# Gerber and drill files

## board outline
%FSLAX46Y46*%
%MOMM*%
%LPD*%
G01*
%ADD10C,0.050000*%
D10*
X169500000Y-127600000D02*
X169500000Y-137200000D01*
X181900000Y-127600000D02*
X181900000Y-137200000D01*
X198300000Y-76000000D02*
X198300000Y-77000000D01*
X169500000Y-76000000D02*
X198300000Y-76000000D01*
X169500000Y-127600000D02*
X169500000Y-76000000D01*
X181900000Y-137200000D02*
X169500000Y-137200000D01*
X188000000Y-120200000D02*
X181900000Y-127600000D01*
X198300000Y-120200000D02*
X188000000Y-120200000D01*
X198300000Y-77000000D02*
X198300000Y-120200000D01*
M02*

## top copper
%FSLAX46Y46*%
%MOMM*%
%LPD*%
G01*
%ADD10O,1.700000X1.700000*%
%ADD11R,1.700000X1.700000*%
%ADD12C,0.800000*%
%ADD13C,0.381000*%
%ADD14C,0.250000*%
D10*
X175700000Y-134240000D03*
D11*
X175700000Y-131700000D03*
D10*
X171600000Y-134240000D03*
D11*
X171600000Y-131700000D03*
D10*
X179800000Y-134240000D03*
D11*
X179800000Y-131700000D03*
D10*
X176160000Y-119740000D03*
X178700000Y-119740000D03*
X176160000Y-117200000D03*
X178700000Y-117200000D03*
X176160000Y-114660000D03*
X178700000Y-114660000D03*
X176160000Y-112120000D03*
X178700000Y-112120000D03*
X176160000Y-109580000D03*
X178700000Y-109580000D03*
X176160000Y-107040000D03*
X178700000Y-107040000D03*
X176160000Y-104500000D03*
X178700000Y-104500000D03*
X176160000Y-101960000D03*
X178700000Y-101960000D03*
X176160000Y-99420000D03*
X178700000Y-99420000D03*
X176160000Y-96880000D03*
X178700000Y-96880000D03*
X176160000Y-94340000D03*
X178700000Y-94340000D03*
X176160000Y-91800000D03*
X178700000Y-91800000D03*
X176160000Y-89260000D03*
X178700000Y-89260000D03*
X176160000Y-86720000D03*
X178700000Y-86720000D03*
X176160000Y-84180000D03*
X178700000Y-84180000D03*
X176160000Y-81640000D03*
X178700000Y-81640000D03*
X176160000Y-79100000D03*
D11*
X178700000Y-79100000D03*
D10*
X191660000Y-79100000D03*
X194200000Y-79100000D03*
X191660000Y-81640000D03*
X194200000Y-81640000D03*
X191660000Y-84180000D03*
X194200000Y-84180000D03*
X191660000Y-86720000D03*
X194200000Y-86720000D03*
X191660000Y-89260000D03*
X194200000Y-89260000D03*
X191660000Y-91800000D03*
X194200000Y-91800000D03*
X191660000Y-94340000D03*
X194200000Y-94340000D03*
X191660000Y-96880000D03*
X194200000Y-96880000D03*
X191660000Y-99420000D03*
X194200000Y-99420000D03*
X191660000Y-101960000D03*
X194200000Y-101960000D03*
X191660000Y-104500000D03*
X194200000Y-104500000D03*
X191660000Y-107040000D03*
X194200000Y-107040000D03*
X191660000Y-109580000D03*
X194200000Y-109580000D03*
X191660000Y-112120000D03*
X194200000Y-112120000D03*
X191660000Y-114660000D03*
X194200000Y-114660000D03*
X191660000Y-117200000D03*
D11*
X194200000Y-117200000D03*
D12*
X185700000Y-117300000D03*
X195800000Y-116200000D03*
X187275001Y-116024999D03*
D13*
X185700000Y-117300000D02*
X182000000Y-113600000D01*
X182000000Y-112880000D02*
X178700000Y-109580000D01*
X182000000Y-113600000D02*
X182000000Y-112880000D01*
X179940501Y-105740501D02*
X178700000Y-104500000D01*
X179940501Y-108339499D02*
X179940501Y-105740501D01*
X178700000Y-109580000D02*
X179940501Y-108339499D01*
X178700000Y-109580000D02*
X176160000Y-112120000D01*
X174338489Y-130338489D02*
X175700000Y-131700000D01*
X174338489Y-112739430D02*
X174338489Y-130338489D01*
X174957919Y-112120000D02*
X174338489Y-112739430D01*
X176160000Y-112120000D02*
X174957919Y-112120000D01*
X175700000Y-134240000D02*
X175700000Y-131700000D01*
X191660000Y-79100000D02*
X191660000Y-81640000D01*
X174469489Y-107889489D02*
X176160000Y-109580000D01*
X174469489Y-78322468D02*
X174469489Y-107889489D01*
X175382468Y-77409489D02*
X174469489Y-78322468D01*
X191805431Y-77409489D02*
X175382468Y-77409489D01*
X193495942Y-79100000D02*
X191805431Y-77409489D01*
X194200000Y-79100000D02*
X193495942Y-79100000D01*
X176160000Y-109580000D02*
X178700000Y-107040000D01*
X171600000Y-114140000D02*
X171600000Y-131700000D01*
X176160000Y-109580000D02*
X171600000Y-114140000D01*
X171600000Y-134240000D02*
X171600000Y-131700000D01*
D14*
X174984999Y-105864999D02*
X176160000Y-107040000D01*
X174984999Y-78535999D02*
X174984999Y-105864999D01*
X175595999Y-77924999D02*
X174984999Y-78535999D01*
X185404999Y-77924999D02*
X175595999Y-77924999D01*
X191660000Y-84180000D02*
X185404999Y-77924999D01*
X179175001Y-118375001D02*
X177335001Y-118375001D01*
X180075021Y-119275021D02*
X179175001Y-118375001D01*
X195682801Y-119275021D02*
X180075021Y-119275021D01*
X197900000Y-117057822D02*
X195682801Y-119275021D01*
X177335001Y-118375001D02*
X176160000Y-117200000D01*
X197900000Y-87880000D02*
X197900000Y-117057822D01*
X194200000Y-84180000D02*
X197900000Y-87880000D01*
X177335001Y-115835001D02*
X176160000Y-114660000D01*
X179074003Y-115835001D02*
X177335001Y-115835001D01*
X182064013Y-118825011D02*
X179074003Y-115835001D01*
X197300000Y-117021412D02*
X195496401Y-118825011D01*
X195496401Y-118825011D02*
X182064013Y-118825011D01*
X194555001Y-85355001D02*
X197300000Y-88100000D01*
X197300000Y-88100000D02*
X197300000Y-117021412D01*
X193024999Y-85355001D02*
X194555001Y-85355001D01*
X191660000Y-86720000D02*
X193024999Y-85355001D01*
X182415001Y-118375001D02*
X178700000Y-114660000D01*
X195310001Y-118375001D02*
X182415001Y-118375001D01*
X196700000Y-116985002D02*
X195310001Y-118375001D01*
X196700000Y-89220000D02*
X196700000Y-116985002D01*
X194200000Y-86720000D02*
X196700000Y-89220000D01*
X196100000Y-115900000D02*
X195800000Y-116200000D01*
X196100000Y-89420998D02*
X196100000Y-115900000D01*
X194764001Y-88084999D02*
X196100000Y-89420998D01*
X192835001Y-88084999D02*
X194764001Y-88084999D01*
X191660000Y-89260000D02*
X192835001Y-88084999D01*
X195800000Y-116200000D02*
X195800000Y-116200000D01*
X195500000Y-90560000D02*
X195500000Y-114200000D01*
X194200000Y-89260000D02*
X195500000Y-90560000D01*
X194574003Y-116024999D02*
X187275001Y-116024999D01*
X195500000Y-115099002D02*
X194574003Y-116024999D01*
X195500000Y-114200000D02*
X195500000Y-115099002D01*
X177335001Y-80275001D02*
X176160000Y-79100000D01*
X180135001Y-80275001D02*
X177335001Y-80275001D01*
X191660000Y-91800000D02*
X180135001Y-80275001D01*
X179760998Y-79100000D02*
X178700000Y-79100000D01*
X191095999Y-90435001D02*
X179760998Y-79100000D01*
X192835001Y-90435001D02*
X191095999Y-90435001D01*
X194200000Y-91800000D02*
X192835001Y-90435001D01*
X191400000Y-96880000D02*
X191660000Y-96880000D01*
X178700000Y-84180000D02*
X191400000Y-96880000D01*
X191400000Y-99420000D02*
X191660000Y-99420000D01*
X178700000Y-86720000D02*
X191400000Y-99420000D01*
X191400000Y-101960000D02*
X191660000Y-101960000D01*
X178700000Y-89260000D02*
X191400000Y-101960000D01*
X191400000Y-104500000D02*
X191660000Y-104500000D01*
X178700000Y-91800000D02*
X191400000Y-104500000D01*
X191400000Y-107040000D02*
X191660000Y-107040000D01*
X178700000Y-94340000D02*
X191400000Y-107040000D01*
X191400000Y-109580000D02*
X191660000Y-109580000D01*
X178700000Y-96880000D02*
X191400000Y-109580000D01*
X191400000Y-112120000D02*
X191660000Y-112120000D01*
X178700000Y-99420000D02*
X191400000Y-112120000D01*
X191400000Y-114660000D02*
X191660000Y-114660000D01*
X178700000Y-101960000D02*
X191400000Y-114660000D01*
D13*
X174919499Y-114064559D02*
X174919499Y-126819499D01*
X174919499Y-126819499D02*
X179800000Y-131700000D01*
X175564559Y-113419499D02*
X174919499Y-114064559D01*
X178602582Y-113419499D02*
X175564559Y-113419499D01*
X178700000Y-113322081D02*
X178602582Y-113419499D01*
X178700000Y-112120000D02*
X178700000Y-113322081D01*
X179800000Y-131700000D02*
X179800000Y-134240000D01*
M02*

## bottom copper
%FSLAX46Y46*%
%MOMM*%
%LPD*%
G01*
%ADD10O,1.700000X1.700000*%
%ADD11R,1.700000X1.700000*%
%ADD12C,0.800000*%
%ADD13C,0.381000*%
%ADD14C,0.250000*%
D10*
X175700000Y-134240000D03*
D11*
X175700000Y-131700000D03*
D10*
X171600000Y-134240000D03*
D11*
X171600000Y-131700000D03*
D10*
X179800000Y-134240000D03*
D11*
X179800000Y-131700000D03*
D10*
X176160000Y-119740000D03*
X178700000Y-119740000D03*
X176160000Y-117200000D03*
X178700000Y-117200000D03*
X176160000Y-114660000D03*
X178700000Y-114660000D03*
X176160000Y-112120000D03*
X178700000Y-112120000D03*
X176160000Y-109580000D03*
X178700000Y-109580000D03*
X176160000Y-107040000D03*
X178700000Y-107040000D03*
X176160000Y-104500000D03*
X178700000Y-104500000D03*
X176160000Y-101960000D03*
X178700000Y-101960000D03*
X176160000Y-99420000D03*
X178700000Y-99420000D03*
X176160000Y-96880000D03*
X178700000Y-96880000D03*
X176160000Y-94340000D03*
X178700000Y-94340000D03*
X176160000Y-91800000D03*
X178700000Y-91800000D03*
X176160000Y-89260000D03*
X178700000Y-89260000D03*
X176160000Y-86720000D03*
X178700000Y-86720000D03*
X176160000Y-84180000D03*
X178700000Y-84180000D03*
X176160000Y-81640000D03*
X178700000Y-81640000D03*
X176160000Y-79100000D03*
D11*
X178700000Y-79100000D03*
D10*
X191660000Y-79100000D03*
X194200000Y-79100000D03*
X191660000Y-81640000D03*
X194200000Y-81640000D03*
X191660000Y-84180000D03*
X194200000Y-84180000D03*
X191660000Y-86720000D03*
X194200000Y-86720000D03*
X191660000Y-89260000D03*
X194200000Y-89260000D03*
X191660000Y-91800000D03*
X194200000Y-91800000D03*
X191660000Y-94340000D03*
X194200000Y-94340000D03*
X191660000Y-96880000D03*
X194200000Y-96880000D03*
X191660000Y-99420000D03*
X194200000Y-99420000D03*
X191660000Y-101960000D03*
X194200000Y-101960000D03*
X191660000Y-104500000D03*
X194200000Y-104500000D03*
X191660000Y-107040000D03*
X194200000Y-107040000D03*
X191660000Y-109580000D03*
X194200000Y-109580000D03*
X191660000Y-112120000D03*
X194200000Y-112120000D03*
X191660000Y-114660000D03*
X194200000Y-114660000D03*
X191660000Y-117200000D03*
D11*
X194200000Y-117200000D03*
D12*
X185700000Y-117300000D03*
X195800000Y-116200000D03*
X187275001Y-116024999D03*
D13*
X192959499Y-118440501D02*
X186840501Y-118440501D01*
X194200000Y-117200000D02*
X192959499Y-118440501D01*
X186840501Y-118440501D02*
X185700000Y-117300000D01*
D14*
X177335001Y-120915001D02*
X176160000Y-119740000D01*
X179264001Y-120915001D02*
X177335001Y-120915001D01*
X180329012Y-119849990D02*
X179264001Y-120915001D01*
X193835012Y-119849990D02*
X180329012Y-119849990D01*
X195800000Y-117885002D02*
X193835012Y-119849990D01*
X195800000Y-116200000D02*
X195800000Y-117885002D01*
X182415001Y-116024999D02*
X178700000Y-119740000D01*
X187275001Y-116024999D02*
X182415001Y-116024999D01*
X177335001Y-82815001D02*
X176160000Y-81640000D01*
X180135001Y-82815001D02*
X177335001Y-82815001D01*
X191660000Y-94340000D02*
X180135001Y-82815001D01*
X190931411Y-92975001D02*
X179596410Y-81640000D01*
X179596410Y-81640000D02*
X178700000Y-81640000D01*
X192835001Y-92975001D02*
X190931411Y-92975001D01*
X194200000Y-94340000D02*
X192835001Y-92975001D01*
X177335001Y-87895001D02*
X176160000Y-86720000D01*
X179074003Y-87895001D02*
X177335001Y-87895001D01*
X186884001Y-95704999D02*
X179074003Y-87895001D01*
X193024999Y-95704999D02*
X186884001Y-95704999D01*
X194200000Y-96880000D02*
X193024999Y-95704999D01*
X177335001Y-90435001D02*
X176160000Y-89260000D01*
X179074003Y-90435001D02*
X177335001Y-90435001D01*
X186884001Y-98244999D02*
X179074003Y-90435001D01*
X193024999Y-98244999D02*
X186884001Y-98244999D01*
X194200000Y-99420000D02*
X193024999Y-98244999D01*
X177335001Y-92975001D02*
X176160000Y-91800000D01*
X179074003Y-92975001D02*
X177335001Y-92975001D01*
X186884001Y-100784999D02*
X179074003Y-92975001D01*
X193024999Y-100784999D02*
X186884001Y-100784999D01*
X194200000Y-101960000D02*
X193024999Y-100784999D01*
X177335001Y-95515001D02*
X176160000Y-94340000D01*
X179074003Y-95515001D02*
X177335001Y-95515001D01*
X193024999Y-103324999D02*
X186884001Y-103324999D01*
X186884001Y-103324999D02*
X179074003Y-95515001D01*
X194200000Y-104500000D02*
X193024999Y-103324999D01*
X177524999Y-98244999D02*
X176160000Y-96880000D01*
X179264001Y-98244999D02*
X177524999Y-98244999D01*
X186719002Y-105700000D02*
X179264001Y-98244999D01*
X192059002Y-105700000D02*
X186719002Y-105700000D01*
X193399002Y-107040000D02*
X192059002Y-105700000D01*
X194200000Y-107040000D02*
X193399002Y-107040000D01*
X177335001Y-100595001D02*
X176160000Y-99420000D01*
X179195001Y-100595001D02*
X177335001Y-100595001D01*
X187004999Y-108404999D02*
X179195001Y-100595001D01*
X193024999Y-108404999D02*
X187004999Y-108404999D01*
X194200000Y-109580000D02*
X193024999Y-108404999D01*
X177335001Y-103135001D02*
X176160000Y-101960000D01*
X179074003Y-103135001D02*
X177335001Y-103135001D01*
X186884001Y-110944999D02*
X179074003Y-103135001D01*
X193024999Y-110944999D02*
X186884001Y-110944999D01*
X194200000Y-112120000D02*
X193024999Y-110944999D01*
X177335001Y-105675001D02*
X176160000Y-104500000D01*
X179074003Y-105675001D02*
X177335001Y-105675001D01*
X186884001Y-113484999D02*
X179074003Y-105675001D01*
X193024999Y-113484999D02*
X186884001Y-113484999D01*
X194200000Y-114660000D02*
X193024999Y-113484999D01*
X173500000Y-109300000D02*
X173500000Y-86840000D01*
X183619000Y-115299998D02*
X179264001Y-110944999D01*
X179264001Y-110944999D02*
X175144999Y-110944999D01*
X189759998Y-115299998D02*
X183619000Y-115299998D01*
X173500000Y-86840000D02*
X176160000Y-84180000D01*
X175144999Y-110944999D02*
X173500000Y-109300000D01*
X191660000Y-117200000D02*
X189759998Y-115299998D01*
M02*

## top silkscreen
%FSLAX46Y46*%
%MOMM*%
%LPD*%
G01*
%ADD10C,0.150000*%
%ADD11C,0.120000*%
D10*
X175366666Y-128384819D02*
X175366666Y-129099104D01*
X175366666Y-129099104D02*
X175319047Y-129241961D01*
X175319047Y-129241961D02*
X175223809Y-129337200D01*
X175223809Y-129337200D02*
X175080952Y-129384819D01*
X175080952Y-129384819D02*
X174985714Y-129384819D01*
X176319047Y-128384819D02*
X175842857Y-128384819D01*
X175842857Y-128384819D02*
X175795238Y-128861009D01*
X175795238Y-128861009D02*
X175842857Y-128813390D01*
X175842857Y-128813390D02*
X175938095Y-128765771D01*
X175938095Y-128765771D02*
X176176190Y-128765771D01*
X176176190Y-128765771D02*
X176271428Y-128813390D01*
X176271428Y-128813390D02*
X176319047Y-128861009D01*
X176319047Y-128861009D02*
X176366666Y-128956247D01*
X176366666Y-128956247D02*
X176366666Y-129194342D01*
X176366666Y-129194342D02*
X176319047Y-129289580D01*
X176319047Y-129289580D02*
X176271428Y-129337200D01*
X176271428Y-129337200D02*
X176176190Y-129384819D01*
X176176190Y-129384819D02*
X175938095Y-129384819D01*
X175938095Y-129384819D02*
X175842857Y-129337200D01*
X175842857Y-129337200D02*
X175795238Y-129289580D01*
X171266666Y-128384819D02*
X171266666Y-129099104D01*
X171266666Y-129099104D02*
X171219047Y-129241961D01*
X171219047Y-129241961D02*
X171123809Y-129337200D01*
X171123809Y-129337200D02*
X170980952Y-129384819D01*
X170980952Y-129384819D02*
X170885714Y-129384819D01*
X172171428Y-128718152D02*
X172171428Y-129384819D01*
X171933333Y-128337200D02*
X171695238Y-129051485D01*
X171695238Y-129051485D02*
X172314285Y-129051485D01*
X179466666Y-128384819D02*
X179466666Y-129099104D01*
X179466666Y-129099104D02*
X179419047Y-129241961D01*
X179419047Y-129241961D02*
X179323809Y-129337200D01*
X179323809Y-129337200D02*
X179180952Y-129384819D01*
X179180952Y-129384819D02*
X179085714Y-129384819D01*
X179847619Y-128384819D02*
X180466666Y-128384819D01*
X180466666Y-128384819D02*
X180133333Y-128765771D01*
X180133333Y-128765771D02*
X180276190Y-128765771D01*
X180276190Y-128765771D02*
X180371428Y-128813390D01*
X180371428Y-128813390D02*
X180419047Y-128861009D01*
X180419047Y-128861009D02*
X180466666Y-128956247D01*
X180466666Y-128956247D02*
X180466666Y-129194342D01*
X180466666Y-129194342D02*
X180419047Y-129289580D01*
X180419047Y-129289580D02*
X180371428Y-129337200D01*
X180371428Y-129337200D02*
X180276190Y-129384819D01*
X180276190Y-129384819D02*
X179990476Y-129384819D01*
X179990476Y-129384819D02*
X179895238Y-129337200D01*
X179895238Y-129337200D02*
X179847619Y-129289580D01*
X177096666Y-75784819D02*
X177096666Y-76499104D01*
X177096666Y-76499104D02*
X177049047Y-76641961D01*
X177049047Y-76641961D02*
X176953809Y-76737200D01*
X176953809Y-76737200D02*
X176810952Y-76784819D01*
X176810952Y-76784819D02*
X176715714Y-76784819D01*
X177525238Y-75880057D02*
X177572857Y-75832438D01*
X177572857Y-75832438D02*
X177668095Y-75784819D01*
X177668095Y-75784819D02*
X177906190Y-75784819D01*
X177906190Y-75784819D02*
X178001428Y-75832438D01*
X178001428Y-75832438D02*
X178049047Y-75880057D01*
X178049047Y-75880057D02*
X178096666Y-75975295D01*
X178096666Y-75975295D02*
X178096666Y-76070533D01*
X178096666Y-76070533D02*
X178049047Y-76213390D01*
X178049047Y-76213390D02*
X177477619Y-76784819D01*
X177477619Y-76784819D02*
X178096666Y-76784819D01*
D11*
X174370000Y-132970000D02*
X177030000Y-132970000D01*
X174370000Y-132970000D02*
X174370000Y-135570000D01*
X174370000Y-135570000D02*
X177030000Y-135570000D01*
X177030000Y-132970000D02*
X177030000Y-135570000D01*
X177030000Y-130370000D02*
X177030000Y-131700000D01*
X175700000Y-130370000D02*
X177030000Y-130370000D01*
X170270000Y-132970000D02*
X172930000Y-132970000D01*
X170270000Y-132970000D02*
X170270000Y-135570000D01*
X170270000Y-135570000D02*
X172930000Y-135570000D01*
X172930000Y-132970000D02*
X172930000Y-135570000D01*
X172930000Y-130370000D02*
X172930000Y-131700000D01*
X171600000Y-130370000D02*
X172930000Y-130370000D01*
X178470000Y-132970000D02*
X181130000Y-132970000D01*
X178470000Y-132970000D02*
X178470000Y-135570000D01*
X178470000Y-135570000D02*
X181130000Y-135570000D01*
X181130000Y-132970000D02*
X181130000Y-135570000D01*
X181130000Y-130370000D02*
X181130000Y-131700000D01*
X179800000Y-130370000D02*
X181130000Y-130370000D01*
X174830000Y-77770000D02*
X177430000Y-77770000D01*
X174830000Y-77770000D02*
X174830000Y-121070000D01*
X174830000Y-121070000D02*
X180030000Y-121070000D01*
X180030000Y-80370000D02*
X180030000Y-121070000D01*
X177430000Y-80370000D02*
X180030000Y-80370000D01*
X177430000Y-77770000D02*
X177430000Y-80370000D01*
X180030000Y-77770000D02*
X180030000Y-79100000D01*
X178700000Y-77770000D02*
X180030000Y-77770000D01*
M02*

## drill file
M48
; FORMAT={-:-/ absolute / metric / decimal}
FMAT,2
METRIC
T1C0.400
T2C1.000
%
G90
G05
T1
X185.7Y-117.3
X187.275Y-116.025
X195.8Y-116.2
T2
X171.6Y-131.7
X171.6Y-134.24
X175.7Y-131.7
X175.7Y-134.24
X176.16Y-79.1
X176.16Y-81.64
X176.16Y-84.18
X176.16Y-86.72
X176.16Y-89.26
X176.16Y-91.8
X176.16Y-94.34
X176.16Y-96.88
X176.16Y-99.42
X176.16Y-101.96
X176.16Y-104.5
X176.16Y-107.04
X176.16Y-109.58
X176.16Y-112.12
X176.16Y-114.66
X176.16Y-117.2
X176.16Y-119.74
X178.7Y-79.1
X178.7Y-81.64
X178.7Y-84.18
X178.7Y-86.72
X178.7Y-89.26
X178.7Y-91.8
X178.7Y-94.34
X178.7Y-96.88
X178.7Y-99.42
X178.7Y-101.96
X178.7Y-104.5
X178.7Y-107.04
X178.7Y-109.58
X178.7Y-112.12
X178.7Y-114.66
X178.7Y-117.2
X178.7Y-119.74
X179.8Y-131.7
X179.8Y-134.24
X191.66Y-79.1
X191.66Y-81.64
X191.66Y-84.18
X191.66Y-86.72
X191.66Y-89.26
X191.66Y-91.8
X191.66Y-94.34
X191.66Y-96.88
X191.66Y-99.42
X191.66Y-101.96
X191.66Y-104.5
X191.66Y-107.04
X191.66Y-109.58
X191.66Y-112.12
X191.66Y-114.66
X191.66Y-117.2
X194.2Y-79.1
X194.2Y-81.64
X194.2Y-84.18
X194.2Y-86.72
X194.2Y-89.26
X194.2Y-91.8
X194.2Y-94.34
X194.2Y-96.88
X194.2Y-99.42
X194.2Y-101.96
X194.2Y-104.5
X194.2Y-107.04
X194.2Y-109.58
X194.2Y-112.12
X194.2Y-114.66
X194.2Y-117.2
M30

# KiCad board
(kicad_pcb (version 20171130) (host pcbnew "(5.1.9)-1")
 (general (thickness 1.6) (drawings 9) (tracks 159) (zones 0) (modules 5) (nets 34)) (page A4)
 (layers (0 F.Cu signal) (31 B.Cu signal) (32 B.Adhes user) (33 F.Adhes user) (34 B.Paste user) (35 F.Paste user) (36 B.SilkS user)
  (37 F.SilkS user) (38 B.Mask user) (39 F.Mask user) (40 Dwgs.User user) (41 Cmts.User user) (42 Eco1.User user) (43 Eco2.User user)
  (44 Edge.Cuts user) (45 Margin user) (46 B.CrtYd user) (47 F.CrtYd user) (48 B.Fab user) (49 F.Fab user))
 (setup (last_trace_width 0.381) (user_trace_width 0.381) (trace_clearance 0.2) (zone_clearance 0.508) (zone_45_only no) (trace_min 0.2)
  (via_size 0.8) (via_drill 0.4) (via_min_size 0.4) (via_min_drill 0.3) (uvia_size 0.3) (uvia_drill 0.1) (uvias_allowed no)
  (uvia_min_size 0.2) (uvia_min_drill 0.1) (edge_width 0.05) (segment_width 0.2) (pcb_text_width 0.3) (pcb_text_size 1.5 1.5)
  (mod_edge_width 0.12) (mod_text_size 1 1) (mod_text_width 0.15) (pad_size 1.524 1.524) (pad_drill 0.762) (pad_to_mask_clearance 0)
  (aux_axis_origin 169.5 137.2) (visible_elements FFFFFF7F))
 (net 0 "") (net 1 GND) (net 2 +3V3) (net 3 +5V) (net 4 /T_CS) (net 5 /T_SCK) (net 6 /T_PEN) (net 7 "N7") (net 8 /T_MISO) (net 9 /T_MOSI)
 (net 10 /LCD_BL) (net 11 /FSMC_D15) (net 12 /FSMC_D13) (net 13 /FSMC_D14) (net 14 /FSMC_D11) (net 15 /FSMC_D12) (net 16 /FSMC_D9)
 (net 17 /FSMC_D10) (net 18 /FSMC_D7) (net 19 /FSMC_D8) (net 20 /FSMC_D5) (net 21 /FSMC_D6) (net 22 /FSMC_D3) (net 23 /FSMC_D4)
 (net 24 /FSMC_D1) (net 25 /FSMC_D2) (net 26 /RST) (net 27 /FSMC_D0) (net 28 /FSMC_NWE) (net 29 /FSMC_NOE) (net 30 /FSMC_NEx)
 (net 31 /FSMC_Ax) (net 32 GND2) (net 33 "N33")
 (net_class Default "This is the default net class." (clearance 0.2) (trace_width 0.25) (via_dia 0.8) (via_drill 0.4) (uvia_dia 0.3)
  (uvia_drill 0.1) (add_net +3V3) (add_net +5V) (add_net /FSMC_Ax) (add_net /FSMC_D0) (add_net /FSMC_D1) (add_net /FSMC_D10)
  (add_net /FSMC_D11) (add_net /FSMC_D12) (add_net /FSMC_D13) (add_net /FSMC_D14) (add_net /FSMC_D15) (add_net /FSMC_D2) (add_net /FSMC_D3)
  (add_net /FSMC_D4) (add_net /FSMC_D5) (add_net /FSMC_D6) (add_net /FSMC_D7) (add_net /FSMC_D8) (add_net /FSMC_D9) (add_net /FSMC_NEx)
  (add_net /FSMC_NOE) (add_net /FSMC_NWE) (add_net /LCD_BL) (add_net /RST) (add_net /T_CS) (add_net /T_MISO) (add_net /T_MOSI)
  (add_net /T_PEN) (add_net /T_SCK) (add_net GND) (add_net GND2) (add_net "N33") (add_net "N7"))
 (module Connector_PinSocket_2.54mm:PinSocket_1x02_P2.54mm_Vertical (layer F.Cu) (at 175.7 131.7)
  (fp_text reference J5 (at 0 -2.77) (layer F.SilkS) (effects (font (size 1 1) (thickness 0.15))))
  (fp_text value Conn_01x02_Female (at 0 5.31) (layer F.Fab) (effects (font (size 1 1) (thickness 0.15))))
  (fp_line (start -1.33 1.27) (end 1.33 1.27) (layer F.SilkS) (width 0.12))
  (fp_line (start -1.33 1.27) (end -1.33 3.87) (layer F.SilkS) (width 0.12))
  (fp_line (start -1.33 3.87) (end 1.33 3.87) (layer F.SilkS) (width 0.12))
  (fp_line (start 1.33 1.27) (end 1.33 3.87) (layer F.SilkS) (width 0.12))
  (fp_line (start 1.33 -1.33) (end 1.33 0) (layer F.SilkS) (width 0.12))
  (fp_line (start 0 -1.33) (end 1.33 -1.33) (layer F.SilkS) (width 0.12))
  (pad 2 thru_hole oval (at 0 2.54) (size 1.7 1.7) (drill 1) (layers *.Cu *.Mask) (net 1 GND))
  (pad 1 thru_hole rect (at 0 0) (size 1.7 1.7) (drill 1) (layers *.Cu *.Mask) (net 1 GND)))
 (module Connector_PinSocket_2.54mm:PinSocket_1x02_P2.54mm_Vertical (layer F.Cu) (at 171.6 131.7)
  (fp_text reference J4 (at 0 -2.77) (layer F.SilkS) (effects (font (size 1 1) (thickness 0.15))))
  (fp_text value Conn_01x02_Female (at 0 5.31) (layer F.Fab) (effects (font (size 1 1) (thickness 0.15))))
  (fp_line (start -1.33 1.27) (end 1.33 1.27) (layer F.SilkS) (width 0.12))
  (fp_line (start -1.33 1.27) (end -1.33 3.87) (layer F.SilkS) (width 0.12))
  (fp_line (start -1.33 3.87) (end 1.33 3.87) (layer F.SilkS) (width 0.12))
  (fp_line (start 1.33 1.27) (end 1.33 3.87) (layer F.SilkS) (width 0.12))
  (fp_line (start 1.33 -1.33) (end 1.33 0) (layer F.SilkS) (width 0.12))
  (fp_line (start 0 -1.33) (end 1.33 -1.33) (layer F.SilkS) (width 0.12))
  (pad 2 thru_hole oval (at 0 2.54) (size 1.7 1.7) (drill 1) (layers *.Cu *.Mask) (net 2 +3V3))
  (pad 1 thru_hole rect (at 0 0) (size 1.7 1.7) (drill 1) (layers *.Cu *.Mask) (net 2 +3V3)))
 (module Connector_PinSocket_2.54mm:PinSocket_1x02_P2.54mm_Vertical (layer F.Cu) (at 179.8 131.7)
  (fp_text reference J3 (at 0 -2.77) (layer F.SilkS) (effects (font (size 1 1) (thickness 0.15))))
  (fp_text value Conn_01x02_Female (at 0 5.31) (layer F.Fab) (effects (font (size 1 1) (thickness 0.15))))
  (fp_line (start -1.33 1.27) (end 1.33 1.27) (layer F.SilkS) (width 0.12))
  (fp_line (start -1.33 1.27) (end -1.33 3.87) (layer F.SilkS) (width 0.12))
  (fp_line (start -1.33 3.87) (end 1.33 3.87) (layer F.SilkS) (width 0.12))
  (fp_line (start 1.33 1.27) (end 1.33 3.87) (layer F.SilkS) (width 0.12))
  (fp_line (start 1.33 -1.33) (end 1.33 0) (layer F.SilkS) (width 0.12))
  (fp_line (start 0 -1.33) (end 1.33 -1.33) (layer F.SilkS) (width 0.12))
  (pad 2 thru_hole oval (at 0 2.54) (size 1.7 1.7) (drill 1) (layers *.Cu *.Mask) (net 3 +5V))
  (pad 1 thru_hole rect (at 0 0) (size 1.7 1.7) (drill 1) (layers *.Cu *.Mask) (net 3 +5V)))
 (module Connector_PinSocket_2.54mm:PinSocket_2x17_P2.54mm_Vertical (layer F.Cu) (at 178.7 79.1)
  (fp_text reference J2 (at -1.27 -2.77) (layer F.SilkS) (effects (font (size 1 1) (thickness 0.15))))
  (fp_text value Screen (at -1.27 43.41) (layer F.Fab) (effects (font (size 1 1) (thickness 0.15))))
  (fp_line (start -3.87 -1.33) (end -1.27 -1.33) (layer F.SilkS) (width 0.12))
  (fp_line (start -3.87 -1.33) (end -3.87 41.97) (layer F.SilkS) (width 0.12))
  (fp_line (start -3.87 41.97) (end 1.33 41.97) (layer F.SilkS) (width 0.12))
  (fp_line (start 1.33 1.27) (end 1.33 41.97) (layer F.SilkS) (width 0.12))
  (fp_line (start -1.27 1.27) (end 1.33 1.27) (layer F.SilkS) (width 0.12))
  (fp_line (start -1.27 -1.33) (end -1.27 1.27) (layer F.SilkS) (width 0.12))
  (fp_line (start 1.33 -1.33) (end 1.33 0) (layer F.SilkS) (width 0.12))
  (fp_line (start 0 -1.33) (end 1.33 -1.33) (layer F.SilkS) (width 0.12))
  (pad 34 thru_hole oval (at -2.54 40.64) (size 1.7 1.7) (drill 1) (layers *.Cu *.Mask) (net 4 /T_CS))
  (pad 33 thru_hole oval (at 0 40.64) (size 1.7 1.7) (drill 1) (layers *.Cu *.Mask) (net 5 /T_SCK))
  (pad 32 thru_hole oval (at -2.54 38.1) (size 1.7 1.7) (drill 1) (layers *.Cu *.Mask) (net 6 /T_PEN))
  (pad 31 thru_hole oval (at 0 38.1) (size 1.7 1.7) (drill 1) (layers *.Cu *.Mask) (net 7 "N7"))
  (pad 30 thru_hole oval (at -2.54 35.56) (size 1.7 1.7) (drill 1) (layers *.Cu *.Mask) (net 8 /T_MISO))
  (pad 29 thru_hole oval (at 0 35.56) (size 1.7 1.7) (drill 1) (layers *.Cu *.Mask) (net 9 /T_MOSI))
  (pad 28 thru_hole oval (at -2.54 33.02) (size 1.7 1.7) (drill 1) (layers *.Cu *.Mask) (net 1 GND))
  (pad 27 thru_hole oval (at 0 33.02) (size 1.7 1.7) (drill 1) (layers *.Cu *.Mask) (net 3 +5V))
  (pad 26 thru_hole oval (at -2.54 30.48) (size 1.7 1.7) (drill 1) (layers *.Cu *.Mask) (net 2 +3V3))
  (pad 25 thru_hole oval (at 0 30.48) (size 1.7 1.7) (drill 1) (layers *.Cu *.Mask) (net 1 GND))
  (pad 24 thru_hole oval (at -2.54 27.94) (size 1.7 1.7) (drill 1) (layers *.Cu *.Mask) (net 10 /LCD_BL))
  (pad 23 thru_hole oval (at 0 27.94) (size 1.7 1.7) (drill 1) (layers *.Cu *.Mask) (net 2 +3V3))
  (pad 22 thru_hole oval (at -2.54 25.4) (size 1.7 1.7) (drill 1) (layers *.Cu *.Mask) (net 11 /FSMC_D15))
  (pad 21 thru_hole oval (at 0 25.4) (size 1.7 1.7) (drill 1) (layers *.Cu *.Mask) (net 1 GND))
  (pad 20 thru_hole oval (at -2.54 22.86) (size 1.7 1.7) (drill 1) (layers *.Cu *.Mask) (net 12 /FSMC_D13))
  (pad 19 thru_hole oval (at 0 22.86) (size 1.7 1.7) (drill 1) (layers *.Cu *.Mask) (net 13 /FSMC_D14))
  (pad 18 thru_hole oval (at -2.54 20.32) (size 1.7 1.7) (drill 1) (layers *.Cu *.Mask) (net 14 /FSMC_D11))
  (pad 17 thru_hole oval (at 0 20.32) (size 1.7 1.7) (drill 1) (layers *.Cu *.Mask) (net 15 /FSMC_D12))
  (pad 16 thru_hole oval (at -2.54 17.78) (size 1.7 1.7) (drill 1) (layers *.Cu *.Mask) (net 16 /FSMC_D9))
  (pad 15 thru_hole oval (at 0 17.78) (size 1.7 1.7) (drill 1) (layers *.Cu *.Mask) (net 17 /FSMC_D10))
  (pad 14 thru_hole oval (at -2.54 15.24) (size 1.7 1.7) (drill 1) (layers *.Cu *.Mask) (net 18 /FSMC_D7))
  (pad 13 thru_hole oval (at 0 15.24) (size 1.7 1.7) (drill 1) (layers *.Cu *.Mask) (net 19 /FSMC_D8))
  (pad 12 thru_hole oval (at -2.54 12.7) (size 1.7 1.7) (drill 1) (layers *.Cu *.Mask) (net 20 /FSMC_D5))
  (pad 11 thru_hole oval (at 0 12.7) (size 1.7 1.7) (drill 1) (layers *.Cu *.Mask) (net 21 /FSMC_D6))
  (pad 10 thru_hole oval (at -2.54 10.16) (size 1.7 1.7) (drill 1) (layers *.Cu *.Mask) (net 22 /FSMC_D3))
  (pad 9 thru_hole oval (at 0 10.16) (size 1.7 1.7) (drill 1) (layers *.Cu *.Mask) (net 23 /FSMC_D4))
  (pad 8 thru_hole oval (at -2.54 7.62) (size 1.7 1.7) (drill 1) (layers *.Cu *.Mask) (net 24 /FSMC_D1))
  (pad 7 thru_hole oval (at 0 7.62) (size 1.7 1.7) (drill 1) (layers *.Cu *.Mask) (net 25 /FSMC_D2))
  (pad 6 thru_hole oval (at -2.54 5.08) (size 1.7 1.7) (drill 1) (layers *.Cu *.Mask) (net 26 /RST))
  (pad 5 thru_hole oval (at 0 5.08) (size 1.7 1.7) (drill 1) (layers *.Cu *.Mask) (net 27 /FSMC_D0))
  (pad 4 thru_hole oval (at -2.54 2.54) (size 1.7 1.7) (drill 1) (layers *.Cu *.Mask) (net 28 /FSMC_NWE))
  (pad 3 thru_hole oval (at 0 2.54) (size 1.7 1.7) (drill 1) (layers *.Cu *.Mask) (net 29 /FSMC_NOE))
  (pad 2 thru_hole oval (at -2.54 0) (size 1.7 1.7) (drill 1) (layers *.Cu *.Mask) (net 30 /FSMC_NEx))
  (pad 1 thru_hole rect (at 0 0) (size 1.7 1.7) (drill 1) (layers *.Cu *.Mask) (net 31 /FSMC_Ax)))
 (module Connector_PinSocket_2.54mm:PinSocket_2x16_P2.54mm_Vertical (layer B.Cu) (at 194.2 117.2)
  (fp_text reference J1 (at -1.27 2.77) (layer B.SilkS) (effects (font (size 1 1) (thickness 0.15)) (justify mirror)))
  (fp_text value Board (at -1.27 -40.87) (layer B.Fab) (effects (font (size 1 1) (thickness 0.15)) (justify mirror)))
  (pad 32 thru_hole oval (at -2.54 -38.1) (size 1.7 1.7) (drill 1) (layers *.Cu *.Mask) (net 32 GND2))
  (pad 31 thru_hole oval (at 0 -38.1) (size 1.7 1.7) (drill 1) (layers *.Cu *.Mask) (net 2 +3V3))
  (pad 30 thru_hole oval (at -2.54 -35.56) (size 1.7 1.7) (drill 1) (layers *.Cu *.Mask) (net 32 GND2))
  (pad 29 thru_hole oval (at 0 -35.56) (size 1.7 1.7) (drill 1) (layers *.Cu *.Mask) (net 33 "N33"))
  (pad 28 thru_hole oval (at -2.54 -33.02) (size 1.7 1.7) (drill 1) (layers *.Cu *.Mask) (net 10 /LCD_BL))
  (pad 27 thru_hole oval (at 0 -33.02) (size 1.7 1.7) (drill 1) (layers *.Cu *.Mask) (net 6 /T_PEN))
  (pad 26 thru_hole oval (at -2.54 -30.48) (size 1.7 1.7) (drill 1) (layers *.Cu *.Mask) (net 8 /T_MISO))
  (pad 25 thru_hole oval (at 0 -30.48) (size 1.7 1.7) (drill 1) (layers *.Cu *.Mask) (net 9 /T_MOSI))
  (pad 24 thru_hole oval (at -2.54 -27.94) (size 1.7 1.7) (drill 1) (layers *.Cu *.Mask) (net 4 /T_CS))
  (pad 23 thru_hole oval (at 0 -27.94) (size 1.7 1.7) (drill 1) (layers *.Cu *.Mask) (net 5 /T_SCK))
  (pad 22 thru_hole oval (at -2.54 -25.4) (size 1.7 1.7) (drill 1) (layers *.Cu *.Mask) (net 30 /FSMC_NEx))
  (pad 21 thru_hole oval (at 0 -25.4) (size 1.7 1.7) (drill 1) (layers *.Cu *.Mask) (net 31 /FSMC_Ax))
  (pad 20 thru_hole oval (at -2.54 -22.86) (size 1.7 1.7) (drill 1) (layers *.Cu *.Mask) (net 28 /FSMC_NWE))
  (pad 19 thru_hole oval (at 0 -22.86) (size 1.7 1.7) (drill 1) (layers *.Cu *.Mask) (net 29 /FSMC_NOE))
  (pad 18 thru_hole oval (at -2.54 -20.32) (size 1.7 1.7) (drill 1) (layers *.Cu *.Mask) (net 27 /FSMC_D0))
  (pad 17 thru_hole oval (at 0 -20.32) (size 1.7 1.7) (drill 1) (layers *.Cu *.Mask) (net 24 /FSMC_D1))
  (pad 16 thru_hole oval (at -2.54 -17.78) (size 1.7 1.7) (drill 1) (layers *.Cu *.Mask) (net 25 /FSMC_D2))
  (pad 15 thru_hole oval (at 0 -17.78) (size 1.7 1.7) (drill 1) (layers *.Cu *.Mask) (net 22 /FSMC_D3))
  (pad 14 thru_hole oval (at -2.54 -15.24) (size 1.7 1.7) (drill 1) (layers *.Cu *.Mask) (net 23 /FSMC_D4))
  (pad 13 thru_hole oval (at 0 -15.24) (size 1.7 1.7) (drill 1) (layers *.Cu *.Mask) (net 20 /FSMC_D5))
  (pad 12 thru_hole oval (at -2.54 -12.7) (size 1.7 1.7) (drill 1) (layers *.Cu *.Mask) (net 21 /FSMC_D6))
  (pad 11 thru_hole oval (at 0 -12.7) (size 1.7 1.7) (drill 1) (layers *.Cu *.Mask) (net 18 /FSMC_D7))
  (pad 10 thru_hole oval (at -2.54 -10.16) (size 1.7 1.7) (drill 1) (layers *.Cu *.Mask) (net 19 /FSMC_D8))
  (pad 9 thru_hole oval (at 0 -10.16) (size 1.7 1.7) (drill 1) (layers *.Cu *.Mask) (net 16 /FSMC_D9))
  (pad 8 thru_hole oval (at -2.54 -7.62) (size 1.7 1.7) (drill 1) (layers *.Cu *.Mask) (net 17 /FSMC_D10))
  (pad 7 thru_hole oval (at 0 -7.62) (size 1.7 1.7) (drill 1) (layers *.Cu *.Mask) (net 14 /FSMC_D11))
  (pad 6 thru_hole oval (at -2.54 -5.08) (size 1.7 1.7) (drill 1) (layers *.Cu *.Mask) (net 15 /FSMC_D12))
  (pad 5 thru_hole oval (at 0 -5.08) (size 1.7 1.7) (drill 1) (layers *.Cu *.Mask) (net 12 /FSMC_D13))
  (pad 4 thru_hole oval (at -2.54 -2.54) (size 1.7 1.7) (drill 1) (layers *.Cu *.Mask) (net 13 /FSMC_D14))
  (pad 3 thru_hole oval (at 0 -2.54) (size 1.7 1.7) (drill 1) (layers *.Cu *.Mask) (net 11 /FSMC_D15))
  (pad 2 thru_hole oval (at -2.54 0) (size 1.7 1.7) (drill 1) (layers *.Cu *.Mask) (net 26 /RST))
  (pad 1 thru_hole rect (at 0 0) (size 1.7 1.7) (drill 1) (layers *.Cu *.Mask) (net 1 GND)))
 (gr_line (start 169.5 127.6) (end 169.5 137.2) (layer Edge.Cuts) (width 0.05))
 (gr_line (start 181.9 127.6) (end 181.9 137.2) (layer Edge.Cuts) (width 0.05))
 (gr_line (start 198.3 76) (end 198.3 77) (layer Edge.Cuts) (width 0.05))
 (gr_line (start 169.5 76) (end 198.3 76) (layer Edge.Cuts) (width 0.05))
 (gr_line (start 169.5 127.6) (end 169.5 76) (layer Edge.Cuts) (width 0.05))
 (gr_line (start 181.9 137.2) (end 169.5 137.2) (layer Edge.Cuts) (width 0.05))
 (gr_line (start 188 120.2) (end 181.9 127.6) (layer Edge.Cuts) (width 0.05))
 (gr_line (start 198.3 120.2) (end 188 120.2) (layer Edge.Cuts) (width 0.05))
 (gr_line (start 198.3 77) (end 198.3 120.2) (layer Edge.Cuts) (width 0.05))
 (segment (start 192.959499 118.440501) (end 186.840501 118.440501) (width 0.381) (layer B.Cu) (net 1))
 (segment (start 194.2 117.2) (end 192.959499 118.440501) (width 0.381) (layer B.Cu) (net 1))
 (via (at 185.7 117.3) (size 0.8) (drill 0.4) (layers F.Cu B.Cu) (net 1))
 (segment (start 186.840501 118.440501) (end 185.7 117.3) (width 0.381) (layer B.Cu) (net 1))
 (segment (start 185.7 117.3) (end 182 113.6) (width 0.381) (layer F.Cu) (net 1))
 (segment (start 182 112.88) (end 178.7 109.58) (width 0.381) (layer F.Cu) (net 1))
 (segment (start 182 113.6) (end 182 112.88) (width 0.381) (layer F.Cu) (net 1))
 (segment (start 179.940501 105.740501) (end 178.7 104.5) (width 0.381) (layer F.Cu) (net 1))
 (segment (start 179.940501 108.339499) (end 179.940501 105.740501) (width 0.381) (layer F.Cu) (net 1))
 (segment (start 178.7 109.58) (end 179.940501 108.339499) (width 0.381) (layer F.Cu) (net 1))
 (segment (start 178.7 109.58) (end 176.16 112.12) (width 0.381) (layer F.Cu) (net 1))
 (segment (start 174.338489 130.338489) (end 175.7 131.7) (width 0.381) (layer F.Cu) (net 1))
 (segment (start 174.338489 112.73943) (end 174.338489 130.338489) (width 0.381) (layer F.Cu) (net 1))
 (segment (start 174.957919 112.12) (end 174.338489 112.73943) (width 0.381) (layer F.Cu) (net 1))
 (segment (start 176.16 112.12) (end 174.957919 112.12) (width 0.381) (layer F.Cu) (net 1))
 (segment (start 175.7 134.24) (end 175.7 131.7) (width 0.381) (layer F.Cu) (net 1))
 (segment (start 191.66 79.1) (end 191.66 81.64) (width 0.381) (layer F.Cu) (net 32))
 (segment (start 174.469489 107.889489) (end 176.16 109.58) (width 0.381) (layer F.Cu) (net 2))
 (segment (start 174.469489 78.322468) (end 174.469489 107.889489) (width 0.381) (layer F.Cu) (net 2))
 (segment (start 175.382468 77.409489) (end 174.469489 78.322468) (width 0.381) (layer F.Cu) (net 2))
 (segment (start 191.805431 77.409489) (end 175.382468 77.409489) (width 0.381) (layer F.Cu) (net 2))
 (segment (start 193.495942 79.1) (end 191.805431 77.409489) (width 0.381) (layer F.Cu) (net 2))
 (segment (start 194.2 79.1) (end 193.495942 79.1) (width 0.381) (layer F.Cu) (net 2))
 (segment (start 176.16 109.58) (end 178.7 107.04) (width 0.381) (layer F.Cu) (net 2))
 (segment (start 171.6 114.14) (end 171.6 131.7) (width 0.381) (layer F.Cu) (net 2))
 (segment (start 176.16 109.58) (end 171.6 114.14) (width 0.381) (layer F.Cu) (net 2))
 (segment (start 171.6 134.24) (end 171.6 131.7) (width 0.381) (layer F.Cu) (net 2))
 (segment (start 174.984999 105.864999) (end 176.16 107.04) (width 0.25) (layer F.Cu) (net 10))
 (segment (start 174.984999 78.535999) (end 174.984999 105.864999) (width 0.25) (layer F.Cu) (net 10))
 (segment (start 175.595999 77.924999) (end 174.984999 78.535999) (width 0.25) (layer F.Cu) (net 10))
 (segment (start 185.404999 77.924999) (end 175.595999 77.924999) (width 0.25) (layer F.Cu) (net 10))
 (segment (start 191.66 84.18) (end 185.404999 77.924999) (width 0.25) (layer F.Cu) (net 10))
 (segment (start 179.175001 118.375001) (end 177.335001 118.375001) (width 0.25) (layer F.Cu) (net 6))
 (segment (start 180.075021 119.275021) (end 179.175001 118.375001) (width 0.25) (layer F.Cu) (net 6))
 (segment (start 195.682801 119.275021) (end 180.075021 119.275021) (width 0.25) (layer F.Cu) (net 6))
 (segment (start 197.9 117.057822) (end 195.682801 119.275021) (width 0.25) (layer F.Cu) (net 6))
 (segment (start 177.335001 118.375001) (end 176.16 117.2) (width 0.25) (layer F.Cu) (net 6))
 (segment (start 197.9 87.88) (end 197.9 117.057822) (width 0.25) (layer F.Cu) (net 6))
 (segment (start 194.2 84.18) (end 197.9 87.88) (width 0.25) (layer F.Cu) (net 6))
 (segment (start 177.335001 115.835001) (end 176.16 114.66) (width 0.25) (layer F.Cu) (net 8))
 (segment (start 179.074003 115.835001) (end 177.335001 115.835001) (width 0.25) (layer F.Cu) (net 8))
 (segment (start 182.064013 118.825011) (end 179.074003 115.835001) (width 0.25) (layer F.Cu) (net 8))
 (segment (start 197.3 117.021412) (end 195.496401 118.825011) (width 0.25) (layer F.Cu) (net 8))
 (segment (start 195.496401 118.825011) (end 182.064013 118.825011) (width 0.25) (layer F.Cu) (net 8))
 (segment (start 194.555001 85.355001) (end 197.3 88.1) (width 0.25) (layer F.Cu) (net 8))
 (segment (start 197.3 88.1) (end 197.3 117.021412) (width 0.25) (layer F.Cu) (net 8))
 (segment (start 193.024999 85.355001) (end 194.555001 85.355001) (width 0.25) (layer F.Cu) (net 8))
 (segment (start 191.66 86.72) (end 193.024999 85.355001) (width 0.25) (layer F.Cu) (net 8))
 (segment (start 182.415001 118.375001) (end 178.7 114.66) (width 0.25) (layer F.Cu) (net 9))
 (segment (start 195.310001 118.375001) (end 182.415001 118.375001) (width 0.25) (layer F.Cu) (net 9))
 (segment (start 196.7 116.985002) (end 195.310001 118.375001) (width 0.25) (layer F.Cu) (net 9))
 (segment (start 196.7 89.22) (end 196.7 116.985002) (width 0.25) (layer F.Cu) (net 9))
 (segment (start 194.2 86.72) (end 196.7 89.22) (width 0.25) (layer F.Cu) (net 9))
 (segment (start 196.1 115.9) (end 195.8 116.2) (width 0.25) (layer F.Cu) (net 4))
 (segment (start 196.1 89.420998) (end 196.1 115.9) (width 0.25) (layer F.Cu) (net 4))
 (segment (start 194.764001 88.084999) (end 196.1 89.420998) (width 0.25) (layer F.Cu) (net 4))
 (segment (start 192.835001 88.084999) (end 194.764001 88.084999) (width 0.25) (layer F.Cu) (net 4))
 (segment (start 191.66 89.26) (end 192.835001 88.084999) (width 0.25) (layer F.Cu) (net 4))
 (segment (start 195.8 116.2) (end 195.8 116.2) (width 0.25) (layer F.Cu) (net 4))
 (via (at 195.8 116.2) (size 0.8) (drill 0.4) (layers F.Cu B.Cu) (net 4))
 (segment (start 177.335001 120.915001) (end 176.16 119.74) (width 0.25) (layer B.Cu) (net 4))
 (segment (start 179.264001 120.915001) (end 177.335001 120.915001) (width 0.25) (layer B.Cu) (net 4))
 (segment (start 180.329012 119.84999) (end 179.264001 120.915001) (width 0.25) (layer B.Cu) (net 4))
 (segment (start 193.835012 119.84999) (end 180.329012 119.84999) (width 0.25) (layer B.Cu) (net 4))
 (segment (start 195.8 117.885002) (end 193.835012 119.84999) (width 0.25) (layer B.Cu) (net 4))
 (segment (start 195.8 116.2) (end 195.8 117.885002) (width 0.25) (layer B.Cu) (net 4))
 (segment (start 195.5 90.56) (end 195.5 114.2) (width 0.25) (layer F.Cu) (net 5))
 (segment (start 194.2 89.26) (end 195.5 90.56) (width 0.25) (layer F.Cu) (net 5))
 (segment (start 194.574003 116.024999) (end 187.275001 116.024999) (width 0.25) (layer F.Cu) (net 5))
 (segment (start 195.5 115.099002) (end 194.574003 116.024999) (width 0.25) (layer F.Cu) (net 5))
 (segment (start 195.5 114.2) (end 195.5 115.099002) (width 0.25) (layer F.Cu) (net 5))
 (via (at 187.275001 116.024999) (size 0.8) (drill 0.4) (layers F.Cu B.Cu) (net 5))
 (segment (start 182.415001 116.024999) (end 178.7 119.74) (width 0.25) (layer B.Cu) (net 5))
 (segment (start 187.275001 116.024999) (end 182.415001 116.024999) (width 0.25) (layer B.Cu) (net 5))
 (segment (start 177.335001 80.275001) (end 176.16 79.1) (width 0.25) (layer F.Cu) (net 30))
 (segment (start 180.135001 80.275001) (end 177.335001 80.275001) (width 0.25) (layer F.Cu) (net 30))
 (segment (start 191.66 91.8) (end 180.135001 80.275001) (width 0.25) (layer F.Cu) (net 30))
 (segment (start 179.760998 79.1) (end 178.7 79.1) (width 0.25) (layer F.Cu) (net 31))
 (segment (start 191.095999 90.435001) (end 179.760998 79.1) (width 0.25) (layer F.Cu) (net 31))
 (segment (start 192.835001 90.435001) (end 191.095999 90.435001) (width 0.25) (layer F.Cu) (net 31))
 (segment (start 194.2 91.8) (end 192.835001 90.435001) (width 0.25) (layer F.Cu) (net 31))
 (segment (start 177.335001 82.815001) (end 176.16 81.64) (width 0.25) (layer B.Cu) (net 28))
 (segment (start 180.135001 82.815001) (end 177.335001 82.815001) (width 0.25) (layer B.Cu) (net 28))
 (segment (start 191.66 94.34) (end 180.135001 82.815001) (width 0.25) (layer B.Cu) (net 28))
 (segment (start 190.931411 92.975001) (end 179.59641 81.64) (width 0.25) (layer B.Cu) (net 29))
 (segment (start 179.59641 81.64) (end 178.7 81.64) (width 0.25) (layer B.Cu) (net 29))
 (segment (start 192.835001 92.975001) (end 190.931411 92.975001) (width 0.25) (layer B.Cu) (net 29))
 (segment (start 194.2 94.34) (end 192.835001 92.975001) (width 0.25) (layer B.Cu) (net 29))
 (segment (start 191.4 96.88) (end 191.66 96.88) (width 0.25) (layer F.Cu) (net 27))
 (segment (start 178.7 84.18) (end 191.4 96.88) (width 0.25) (layer F.Cu) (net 27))
 (segment (start 177.335001 87.895001) (end 176.16 86.72) (width 0.25) (layer B.Cu) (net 24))
 (segment (start 179.074003 87.895001) (end 177.335001 87.895001) (width 0.25) (layer B.Cu) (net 24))
 (segment (start 186.884001 95.704999) (end 179.074003 87.895001) (width 0.25) (layer B.Cu) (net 24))
 (segment (start 193.024999 95.704999) (end 186.884001 95.704999) (width 0.25) (layer B.Cu) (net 24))
 (segment (start 194.2 96.88) (end 193.024999 95.704999) (width 0.25) (layer B.Cu) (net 24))
 (segment (start 191.4 99.42) (end 191.66 99.42) (width 0.25) (layer F.Cu) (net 25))
 (segment (start 178.7 86.72) (end 191.4 99.42) (width 0.25) (layer F.Cu) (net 25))
 (segment (start 177.335001 90.435001) (end 176.16 89.26) (width 0.25) (layer B.Cu) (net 22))
 (segment (start 179.074003 90.435001) (end 177.335001 90.435001) (width 0.25) (layer B.Cu) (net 22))
 (segment (start 186.884001 98.244999) (end 179.074003 90.435001) (width 0.25) (layer B.Cu) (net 22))
 (segment (start 193.024999 98.244999) (end 186.884001 98.244999) (width 0.25) (layer B.Cu) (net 22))
 (segment (start 194.2 99.42) (end 193.024999 98.244999) (width 0.25) (layer B.Cu) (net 22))
 (segment (start 191.4 101.96) (end 191.66 101.96) (width 0.25) (layer F.Cu) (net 23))
 (segment (start 178.7 89.26) (end 191.4 101.96) (width 0.25) (layer F.Cu) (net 23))
 (segment (start 177.335001 92.975001) (end 176.16 91.8) (width 0.25) (layer B.Cu) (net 20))
 (segment (start 179.074003 92.975001) (end 177.335001 92.975001) (width 0.25) (layer B.Cu) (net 20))
 (segment (start 186.884001 100.784999) (end 179.074003 92.975001) (width 0.25) (layer B.Cu) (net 20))
 (segment (start 193.024999 100.784999) (end 186.884001 100.784999) (width 0.25) (layer B.Cu) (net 20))
 (segment (start 194.2 101.96) (end 193.024999 100.784999) (width 0.25) (layer B.Cu) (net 20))
 (segment (start 191.4 104.5) (end 191.66 104.5) (width 0.25) (layer F.Cu) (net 21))
 (segment (start 178.7 91.8) (end 191.4 104.5) (width 0.25) (layer F.Cu) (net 21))
 (segment (start 177.335001 95.515001) (end 176.16 94.34) (width 0.25) (layer B.Cu) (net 18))
 (segment (start 179.074003 95.515001) (end 177.335001 95.515001) (width 0.25) (layer B.Cu) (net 18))
 (segment (start 193.024999 103.324999) (end 186.884001 103.324999) (width 0.25) (layer B.Cu) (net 18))
 (segment (start 186.884001 103.324999) (end 179.074003 95.515001) (width 0.25) (layer B.Cu) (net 18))
 (segment (start 194.2 104.5) (end 193.024999 103.324999) (width 0.25) (layer B.Cu) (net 18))
 (segment (start 191.4 107.04) (end 191.66 107.04) (width 0.25) (layer F.Cu) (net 19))
 (segment (start 178.7 94.34) (end 191.4 107.04) (width 0.25) (layer F.Cu) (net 19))
 (segment (start 177.524999 98.244999) (end 176.16 96.88) (width 0.25) (layer B.Cu) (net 16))
 (segment (start 179.264001 98.244999) (end 177.524999 98.244999) (width 0.25) (layer B.Cu) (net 16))
 (segment (start 186.719002 105.7) (end 179.264001 98.244999) (width 0.25) (layer B.Cu) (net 16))
 (segment (start 192.059002 105.7) (end 186.719002 105.7) (width 0.25) (layer B.Cu) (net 16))
 (segment (start 193.399002 107.04) (end 192.059002 105.7) (width 0.25) (layer B.Cu) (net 16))
 (segment (start 194.2 107.04) (end 193.399002 107.04) (width 0.25) (layer B.Cu) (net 16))
 (segment (start 191.4 109.58) (end 191.66 109.58) (width 0.25) (layer F.Cu) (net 17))
 (segment (start 178.7 96.88) (end 191.4 109.58) (width 0.25) (layer F.Cu) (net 17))
 (segment (start 177.335001 100.595001) (end 176.16 99.42) (width 0.25) (layer B.Cu) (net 14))
 (segment (start 179.195001 100.595001) (end 177.335001 100.595001) (width 0.25) (layer B.Cu) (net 14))
 (segment (start 187.004999 108.404999) (end 179.195001 100.595001) (width 0.25) (layer B.Cu) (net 14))
 (segment (start 193.024999 108.404999) (end 187.004999 108.404999) (width 0.25) (layer B.Cu) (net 14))
 (segment (start 194.2 109.58) (end 193.024999 108.404999) (width 0.25) (layer B.Cu) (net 14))
 (segment (start 191.4 112.12) (end 191.66 112.12) (width 0.25) (layer F.Cu) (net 15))
 (segment (start 178.7 99.42) (end 191.4 112.12) (width 0.25) (layer F.Cu) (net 15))
 (segment (start 177.335001 103.135001) (end 176.16 101.96) (width 0.25) (layer B.Cu) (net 12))
 (segment (start 179.074003 103.135001) (end 177.335001 103.135001) (width 0.25) (layer B.Cu) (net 12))
 (segment (start 186.884001 110.944999) (end 179.074003 103.135001) (width 0.25) (layer B.Cu) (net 12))
 (segment (start 193.024999 110.944999) (end 186.884001 110.944999) (width 0.25) (layer B.Cu) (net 12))
 (segment (start 194.2 112.12) (end 193.024999 110.944999) (width 0.25) (layer B.Cu) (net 12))
 (segment (start 191.4 114.66) (end 191.66 114.66) (width 0.25) (layer F.Cu) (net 13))
 (segment (start 178.7 101.96) (end 191.4 114.66) (width 0.25) (layer F.Cu) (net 13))
 (segment (start 177.335001 105.675001) (end 176.16 104.5) (width 0.25) (layer B.Cu) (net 11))
 (segment (start 179.074003 105.675001) (end 177.335001 105.675001) (width 0.25) (layer B.Cu) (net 11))
 (segment (start 186.884001 113.484999) (end 179.074003 105.675001) (width 0.25) (layer B.Cu) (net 11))
 (segment (start 193.024999 113.484999) (end 186.884001 113.484999) (width 0.25) (layer B.Cu) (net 11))
 (segment (start 194.2 114.66) (end 193.024999 113.484999) (width 0.25) (layer B.Cu) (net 11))
 (segment (start 173.5 109.3) (end 173.5 86.84) (width 0.25) (layer B.Cu) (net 26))
 (segment (start 183.619 115.299998) (end 179.264001 110.944999) (width 0.25) (layer B.Cu) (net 26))
 (segment (start 179.264001 110.944999) (end 175.144999 110.944999) (width 0.25) (layer B.Cu) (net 26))
 (segment (start 189.759998 115.299998) (end 183.619 115.299998) (width 0.25) (layer B.Cu) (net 26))
 (segment (start 173.5 86.84) (end 176.16 84.18) (width 0.25) (layer B.Cu) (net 26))
 (segment (start 175.144999 110.944999) (end 173.5 109.3) (width 0.25) (layer B.Cu) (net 26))
 (segment (start 191.66 117.2) (end 189.759998 115.299998) (width 0.25) (layer B.Cu) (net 26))
 (segment (start 174.919499 114.064559) (end 174.919499 126.819499) (width 0.381) (layer F.Cu) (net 3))
 (segment (start 174.919499 126.819499) (end 179.8 131.7) (width 0.381) (layer F.Cu) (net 3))
 (segment (start 175.564559 113.419499) (end 174.919499 114.064559) (width 0.381) (layer F.Cu) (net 3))
 (segment (start 178.602582 113.419499) (end 175.564559 113.419499) (width 0.381) (layer F.Cu) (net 3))
 (segment (start 178.7 113.322081) (end 178.602582 113.419499) (width 0.381) (layer F.Cu) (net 3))
 (segment (start 178.7 112.12) (end 178.7 113.322081) (width 0.381) (layer F.Cu) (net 3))
 (segment (start 179.8 131.7) (end 179.8 134.24) (width 0.381) (layer F.Cu) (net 3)))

